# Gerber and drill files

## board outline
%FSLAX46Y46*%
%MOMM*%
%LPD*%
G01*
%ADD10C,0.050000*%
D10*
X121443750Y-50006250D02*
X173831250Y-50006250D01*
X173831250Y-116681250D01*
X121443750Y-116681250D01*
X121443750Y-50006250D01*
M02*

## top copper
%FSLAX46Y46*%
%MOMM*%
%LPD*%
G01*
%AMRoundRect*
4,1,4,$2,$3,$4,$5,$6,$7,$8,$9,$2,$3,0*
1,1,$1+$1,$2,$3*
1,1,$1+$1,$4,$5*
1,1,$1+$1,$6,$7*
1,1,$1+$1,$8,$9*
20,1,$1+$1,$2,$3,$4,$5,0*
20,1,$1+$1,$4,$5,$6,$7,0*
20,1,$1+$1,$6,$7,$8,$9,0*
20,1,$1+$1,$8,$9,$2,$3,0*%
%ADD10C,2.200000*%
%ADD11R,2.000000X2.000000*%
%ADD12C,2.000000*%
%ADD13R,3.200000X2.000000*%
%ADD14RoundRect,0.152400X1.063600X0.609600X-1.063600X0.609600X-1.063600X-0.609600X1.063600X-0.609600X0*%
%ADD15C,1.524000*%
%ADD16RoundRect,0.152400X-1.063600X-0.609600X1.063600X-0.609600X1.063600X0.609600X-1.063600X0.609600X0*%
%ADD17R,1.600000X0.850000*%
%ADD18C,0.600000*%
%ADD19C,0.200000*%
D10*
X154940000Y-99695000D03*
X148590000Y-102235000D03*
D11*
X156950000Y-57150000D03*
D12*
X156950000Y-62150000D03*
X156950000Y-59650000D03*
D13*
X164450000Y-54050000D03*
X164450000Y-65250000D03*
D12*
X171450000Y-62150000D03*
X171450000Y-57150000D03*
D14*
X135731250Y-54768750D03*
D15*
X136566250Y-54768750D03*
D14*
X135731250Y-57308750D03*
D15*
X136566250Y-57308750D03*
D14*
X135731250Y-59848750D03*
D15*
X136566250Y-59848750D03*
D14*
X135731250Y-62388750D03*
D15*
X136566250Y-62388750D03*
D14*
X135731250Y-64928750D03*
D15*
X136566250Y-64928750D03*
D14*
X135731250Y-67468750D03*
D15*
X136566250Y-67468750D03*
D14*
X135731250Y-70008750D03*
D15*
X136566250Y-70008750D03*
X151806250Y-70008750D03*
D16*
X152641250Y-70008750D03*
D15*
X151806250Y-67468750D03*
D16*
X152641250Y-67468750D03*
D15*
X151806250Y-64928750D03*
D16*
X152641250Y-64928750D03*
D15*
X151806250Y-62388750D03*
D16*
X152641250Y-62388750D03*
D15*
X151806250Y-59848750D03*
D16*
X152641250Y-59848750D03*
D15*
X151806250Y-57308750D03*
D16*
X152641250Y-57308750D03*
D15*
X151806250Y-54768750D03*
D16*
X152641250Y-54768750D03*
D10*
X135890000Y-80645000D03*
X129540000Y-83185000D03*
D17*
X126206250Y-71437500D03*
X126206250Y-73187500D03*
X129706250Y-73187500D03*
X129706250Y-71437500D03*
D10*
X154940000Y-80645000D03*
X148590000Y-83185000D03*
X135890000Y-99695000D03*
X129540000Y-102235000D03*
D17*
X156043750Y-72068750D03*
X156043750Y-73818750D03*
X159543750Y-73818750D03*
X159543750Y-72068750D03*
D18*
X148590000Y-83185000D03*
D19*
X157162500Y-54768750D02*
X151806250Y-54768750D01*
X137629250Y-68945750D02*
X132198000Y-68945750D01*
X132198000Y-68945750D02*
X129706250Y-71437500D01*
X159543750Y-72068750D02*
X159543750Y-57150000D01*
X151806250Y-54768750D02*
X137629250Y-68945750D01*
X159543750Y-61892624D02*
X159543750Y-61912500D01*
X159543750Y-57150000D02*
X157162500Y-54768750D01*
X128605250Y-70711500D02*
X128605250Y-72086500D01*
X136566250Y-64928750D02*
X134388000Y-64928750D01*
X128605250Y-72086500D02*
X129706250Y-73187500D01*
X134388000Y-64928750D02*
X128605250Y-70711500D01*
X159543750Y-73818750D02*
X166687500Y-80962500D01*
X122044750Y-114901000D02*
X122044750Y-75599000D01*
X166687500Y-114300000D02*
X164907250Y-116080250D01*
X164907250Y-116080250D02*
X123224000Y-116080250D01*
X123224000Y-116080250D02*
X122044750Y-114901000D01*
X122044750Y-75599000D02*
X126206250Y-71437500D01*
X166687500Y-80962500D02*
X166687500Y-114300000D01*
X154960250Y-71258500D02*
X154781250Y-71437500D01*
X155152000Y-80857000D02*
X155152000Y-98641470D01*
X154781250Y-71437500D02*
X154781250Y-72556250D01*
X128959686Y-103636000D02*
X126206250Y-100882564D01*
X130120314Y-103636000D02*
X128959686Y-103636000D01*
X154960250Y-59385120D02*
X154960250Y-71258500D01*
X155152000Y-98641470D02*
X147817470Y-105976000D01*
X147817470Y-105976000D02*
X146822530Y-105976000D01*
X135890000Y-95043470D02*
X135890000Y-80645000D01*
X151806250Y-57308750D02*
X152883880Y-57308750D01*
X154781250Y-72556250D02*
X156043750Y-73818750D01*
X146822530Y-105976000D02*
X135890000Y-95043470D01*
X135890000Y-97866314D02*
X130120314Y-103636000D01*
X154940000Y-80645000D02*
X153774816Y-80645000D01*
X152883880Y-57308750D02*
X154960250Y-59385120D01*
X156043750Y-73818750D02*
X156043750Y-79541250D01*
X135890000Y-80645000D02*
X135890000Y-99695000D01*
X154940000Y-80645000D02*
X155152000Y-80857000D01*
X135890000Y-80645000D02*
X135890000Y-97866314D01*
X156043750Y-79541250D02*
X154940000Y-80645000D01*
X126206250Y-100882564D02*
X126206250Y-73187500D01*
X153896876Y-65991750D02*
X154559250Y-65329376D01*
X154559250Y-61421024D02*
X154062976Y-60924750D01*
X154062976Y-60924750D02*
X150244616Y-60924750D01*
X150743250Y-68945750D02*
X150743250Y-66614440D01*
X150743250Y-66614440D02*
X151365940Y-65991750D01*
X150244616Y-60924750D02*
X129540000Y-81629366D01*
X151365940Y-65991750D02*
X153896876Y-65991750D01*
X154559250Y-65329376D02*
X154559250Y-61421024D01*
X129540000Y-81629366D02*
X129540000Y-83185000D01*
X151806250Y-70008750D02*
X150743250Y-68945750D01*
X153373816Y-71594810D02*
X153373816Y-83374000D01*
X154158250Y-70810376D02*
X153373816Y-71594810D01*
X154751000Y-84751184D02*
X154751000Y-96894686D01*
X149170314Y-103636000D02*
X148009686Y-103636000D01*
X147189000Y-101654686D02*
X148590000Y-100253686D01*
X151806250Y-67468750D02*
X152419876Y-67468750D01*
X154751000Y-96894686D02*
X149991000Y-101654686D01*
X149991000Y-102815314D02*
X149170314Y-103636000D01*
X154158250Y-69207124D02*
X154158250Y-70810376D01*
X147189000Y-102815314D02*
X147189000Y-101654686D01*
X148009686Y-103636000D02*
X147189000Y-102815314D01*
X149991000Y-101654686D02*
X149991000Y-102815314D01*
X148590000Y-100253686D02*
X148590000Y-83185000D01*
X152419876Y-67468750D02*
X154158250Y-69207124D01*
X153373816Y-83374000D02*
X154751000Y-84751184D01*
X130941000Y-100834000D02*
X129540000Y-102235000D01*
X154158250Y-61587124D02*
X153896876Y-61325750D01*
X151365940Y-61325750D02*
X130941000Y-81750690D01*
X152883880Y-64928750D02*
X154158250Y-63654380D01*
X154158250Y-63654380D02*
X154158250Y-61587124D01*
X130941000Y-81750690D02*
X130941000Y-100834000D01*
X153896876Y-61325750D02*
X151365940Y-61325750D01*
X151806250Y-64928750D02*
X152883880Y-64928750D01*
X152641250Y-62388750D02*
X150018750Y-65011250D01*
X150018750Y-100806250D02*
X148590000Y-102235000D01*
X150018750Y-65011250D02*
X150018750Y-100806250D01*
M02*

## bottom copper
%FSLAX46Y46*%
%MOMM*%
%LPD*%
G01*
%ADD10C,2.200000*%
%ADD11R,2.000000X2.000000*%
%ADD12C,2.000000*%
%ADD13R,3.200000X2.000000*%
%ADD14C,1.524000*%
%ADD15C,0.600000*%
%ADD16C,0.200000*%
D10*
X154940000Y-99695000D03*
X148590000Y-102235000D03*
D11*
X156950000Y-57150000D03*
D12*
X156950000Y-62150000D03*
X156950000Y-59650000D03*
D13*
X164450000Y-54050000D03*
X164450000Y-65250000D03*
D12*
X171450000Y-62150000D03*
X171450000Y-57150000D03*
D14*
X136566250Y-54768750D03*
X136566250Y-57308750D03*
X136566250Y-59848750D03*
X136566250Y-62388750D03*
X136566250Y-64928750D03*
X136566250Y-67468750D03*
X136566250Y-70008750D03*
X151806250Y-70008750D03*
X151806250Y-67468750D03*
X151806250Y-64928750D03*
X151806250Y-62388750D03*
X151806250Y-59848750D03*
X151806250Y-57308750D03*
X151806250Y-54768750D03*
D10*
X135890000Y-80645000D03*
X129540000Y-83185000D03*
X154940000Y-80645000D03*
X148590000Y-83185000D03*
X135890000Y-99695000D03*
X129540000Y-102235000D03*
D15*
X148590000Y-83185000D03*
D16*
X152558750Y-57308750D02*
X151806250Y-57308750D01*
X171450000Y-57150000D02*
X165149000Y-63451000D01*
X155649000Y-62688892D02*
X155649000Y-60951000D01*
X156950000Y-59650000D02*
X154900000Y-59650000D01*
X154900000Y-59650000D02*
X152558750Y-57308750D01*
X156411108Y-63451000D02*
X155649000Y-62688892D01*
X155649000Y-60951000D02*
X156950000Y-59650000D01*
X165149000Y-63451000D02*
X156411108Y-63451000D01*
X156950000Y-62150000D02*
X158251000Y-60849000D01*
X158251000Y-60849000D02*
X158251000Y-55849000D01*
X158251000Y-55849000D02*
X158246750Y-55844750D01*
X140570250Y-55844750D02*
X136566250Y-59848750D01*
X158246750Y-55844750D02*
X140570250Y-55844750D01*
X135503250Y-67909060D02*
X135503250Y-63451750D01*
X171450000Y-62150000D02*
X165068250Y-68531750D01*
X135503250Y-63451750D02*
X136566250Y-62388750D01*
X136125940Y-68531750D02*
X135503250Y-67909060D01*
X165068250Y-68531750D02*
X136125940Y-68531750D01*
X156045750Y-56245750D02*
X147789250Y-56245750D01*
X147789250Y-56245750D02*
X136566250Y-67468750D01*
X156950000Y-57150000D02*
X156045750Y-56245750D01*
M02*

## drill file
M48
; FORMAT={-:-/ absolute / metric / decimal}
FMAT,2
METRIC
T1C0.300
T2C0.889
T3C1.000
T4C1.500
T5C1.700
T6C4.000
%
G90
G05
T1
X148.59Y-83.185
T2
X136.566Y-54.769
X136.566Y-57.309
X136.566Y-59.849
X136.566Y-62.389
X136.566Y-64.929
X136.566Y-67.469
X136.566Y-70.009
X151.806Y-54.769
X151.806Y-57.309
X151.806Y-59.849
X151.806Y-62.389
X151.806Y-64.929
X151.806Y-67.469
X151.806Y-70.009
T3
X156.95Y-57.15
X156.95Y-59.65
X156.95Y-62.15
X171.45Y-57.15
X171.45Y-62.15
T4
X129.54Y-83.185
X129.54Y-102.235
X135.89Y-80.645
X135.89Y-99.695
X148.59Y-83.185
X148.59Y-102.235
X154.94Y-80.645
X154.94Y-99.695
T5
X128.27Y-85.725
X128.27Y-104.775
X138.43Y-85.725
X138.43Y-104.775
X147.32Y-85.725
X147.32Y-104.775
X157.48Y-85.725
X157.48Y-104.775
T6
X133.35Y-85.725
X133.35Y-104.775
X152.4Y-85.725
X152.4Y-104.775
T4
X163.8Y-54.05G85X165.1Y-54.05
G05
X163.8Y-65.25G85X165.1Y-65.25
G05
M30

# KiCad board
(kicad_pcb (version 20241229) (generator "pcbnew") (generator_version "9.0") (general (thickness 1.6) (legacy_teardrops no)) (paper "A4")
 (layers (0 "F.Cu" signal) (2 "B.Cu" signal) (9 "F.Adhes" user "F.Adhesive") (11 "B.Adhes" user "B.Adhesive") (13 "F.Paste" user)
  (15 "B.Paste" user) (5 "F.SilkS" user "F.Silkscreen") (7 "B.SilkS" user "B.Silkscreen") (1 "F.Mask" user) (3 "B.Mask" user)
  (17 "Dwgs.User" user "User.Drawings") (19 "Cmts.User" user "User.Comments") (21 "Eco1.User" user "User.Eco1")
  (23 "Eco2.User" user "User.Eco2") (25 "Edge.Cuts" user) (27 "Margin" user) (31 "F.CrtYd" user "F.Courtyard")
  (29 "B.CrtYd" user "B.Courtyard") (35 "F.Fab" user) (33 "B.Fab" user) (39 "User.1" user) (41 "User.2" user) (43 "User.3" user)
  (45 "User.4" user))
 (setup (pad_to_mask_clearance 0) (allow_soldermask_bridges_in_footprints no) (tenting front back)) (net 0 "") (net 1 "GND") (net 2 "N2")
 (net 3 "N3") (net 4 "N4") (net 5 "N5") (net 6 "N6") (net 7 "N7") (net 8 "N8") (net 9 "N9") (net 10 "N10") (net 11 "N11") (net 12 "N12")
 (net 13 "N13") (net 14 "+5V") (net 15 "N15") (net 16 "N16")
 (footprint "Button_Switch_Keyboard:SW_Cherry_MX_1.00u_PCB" (layer "F.Cu") (at 154.94 99.695)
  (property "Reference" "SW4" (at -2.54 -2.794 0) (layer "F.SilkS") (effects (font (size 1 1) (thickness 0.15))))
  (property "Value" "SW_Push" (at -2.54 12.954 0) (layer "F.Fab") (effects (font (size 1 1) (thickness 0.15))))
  (pad "" np_thru_hole circle (at -7.62 5.08) (size 1.7 1.7) (drill 1.7) (layers "*.Cu" "*.Mask"))
  (pad "" np_thru_hole circle (at -2.54 5.08) (size 4 4) (drill 4) (layers "*.Cu" "*.Mask"))
  (pad "" np_thru_hole circle (at 2.54 5.08) (size 1.7 1.7) (drill 1.7) (layers "*.Cu" "*.Mask"))
  (pad "1" thru_hole circle (at 0 0) (size 2.2 2.2) (drill 1.5) (layers "*.Cu" "*.Mask") (remove_unused_layers no) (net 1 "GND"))
  (pad "2" thru_hole circle (at -6.35 2.54) (size 2.2 2.2) (drill 1.5) (layers "*.Cu" "*.Mask") (remove_unused_layers no) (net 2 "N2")))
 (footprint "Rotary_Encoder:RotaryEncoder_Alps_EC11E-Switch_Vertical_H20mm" (layer "F.Cu") (at 156.95 57.15)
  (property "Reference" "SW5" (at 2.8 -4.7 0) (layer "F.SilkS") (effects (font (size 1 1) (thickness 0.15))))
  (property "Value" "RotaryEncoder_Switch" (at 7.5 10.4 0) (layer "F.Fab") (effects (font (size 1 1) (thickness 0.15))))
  (pad "A" thru_hole rect (at 0 0) (size 2 2) (drill 1) (layers "*.Cu" "*.Mask") (remove_unused_layers no) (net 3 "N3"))
  (pad "B" thru_hole circle (at 0 5) (size 2 2) (drill 1) (layers "*.Cu" "*.Mask") (remove_unused_layers no) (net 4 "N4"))
  (pad "C" thru_hole circle (at 0 2.5) (size 2 2) (drill 1) (layers "*.Cu" "*.Mask") (remove_unused_layers no) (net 1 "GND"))
  (pad "MP" thru_hole rect (at 7.5 -3.1) (size 3.2 2) (drill oval 2.8 1.5) (layers "*.Cu" "*.Mask") (remove_unused_layers no))
  (pad "MP" thru_hole rect (at 7.5 8.1) (size 3.2 2) (drill oval 2.8 1.5) (layers "*.Cu" "*.Mask") (remove_unused_layers no))
  (pad "S1" thru_hole circle (at 14.5 5) (size 2 2) (drill 1) (layers "*.Cu" "*.Mask") (remove_unused_layers no) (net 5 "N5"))
  (pad "S2" thru_hole circle (at 14.5 0) (size 2 2) (drill 1) (layers "*.Cu" "*.Mask") (remove_unused_layers no) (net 1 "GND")))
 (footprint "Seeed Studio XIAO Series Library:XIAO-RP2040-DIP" (layer "F.Cu") (at 144.18625 62.38875)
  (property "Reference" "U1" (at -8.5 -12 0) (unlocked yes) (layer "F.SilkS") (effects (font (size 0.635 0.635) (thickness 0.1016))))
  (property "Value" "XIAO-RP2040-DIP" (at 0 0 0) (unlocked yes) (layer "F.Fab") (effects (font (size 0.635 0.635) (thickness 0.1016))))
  (pad "1" smd roundrect (at -8.455 -7.62 180) (size 2.432 1.524) (layers "F.Cu" "F.Mask") (roundrect_rratio 0.1) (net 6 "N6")
   (thermal_bridge_angle 45))
  (pad "1" thru_hole circle (at -7.62 -7.62 180) (size 1.524 1.524) (drill 0.889) (layers "*.Cu" "*.Mask") (remove_unused_layers no)
   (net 6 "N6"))
  (pad "2" smd roundrect (at -8.455 -5.08 180) (size 2.432 1.524) (layers "F.Cu" "F.Mask") (roundrect_rratio 0.1) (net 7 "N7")
   (thermal_bridge_angle 45))
  (pad "2" thru_hole circle (at -7.62 -5.08 180) (size 1.524 1.524) (drill 0.889) (layers "*.Cu" "*.Mask") (remove_unused_layers no)
   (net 7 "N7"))
  (pad "3" smd roundrect (at -8.455 -2.54 180) (size 2.432 1.524) (layers "F.Cu" "F.Mask") (roundrect_rratio 0.1) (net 4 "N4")
   (thermal_bridge_angle 45))
  (pad "3" thru_hole circle (at -7.62 -2.54 180) (size 1.524 1.524) (drill 0.889) (layers "*.Cu" "*.Mask") (remove_unused_layers no)
   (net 4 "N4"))
  (pad "4" smd roundrect (at -8.455 0 180) (size 2.432 1.524) (layers "F.Cu" "F.Mask") (roundrect_rratio 0.1) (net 5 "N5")
   (thermal_bridge_angle 45))
  (pad "4" thru_hole circle (at -7.62 0 180) (size 1.524 1.524) (drill 0.889) (layers "*.Cu" "*.Mask") (remove_unused_layers no)
   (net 5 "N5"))
  (pad "5" smd roundrect (at -8.455 2.54 180) (size 2.432 1.524) (layers "F.Cu" "F.Mask") (roundrect_rratio 0.1) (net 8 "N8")
   (thermal_bridge_angle 45))
  (pad "5" thru_hole circle (at -7.62 2.54 180) (size 1.524 1.524) (drill 0.889) (layers "*.Cu" "*.Mask") (remove_unused_layers no)
   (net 8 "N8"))
  (pad "6" smd roundrect (at -8.455 5.08 180) (size 2.432 1.524) (layers "F.Cu" "F.Mask") (roundrect_rratio 0.1) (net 3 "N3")
   (thermal_bridge_angle 45))
  (pad "6" thru_hole circle (at -7.62 5.08 180) (size 1.524 1.524) (drill 0.889) (layers "*.Cu" "*.Mask") (remove_unused_layers no)
   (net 3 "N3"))
  (pad "7" smd roundrect (at -8.455 7.62 180) (size 2.432 1.524) (layers "F.Cu" "F.Mask") (roundrect_rratio 0.1) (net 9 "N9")
   (thermal_bridge_angle 45))
  (pad "7" thru_hole circle (at -7.62 7.62 180) (size 1.524 1.524) (drill 0.889) (layers "*.Cu" "*.Mask") (remove_unused_layers no)
   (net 9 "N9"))
  (pad "8" thru_hole circle (at 7.62 7.62) (size 1.524 1.524) (drill 0.889) (layers "*.Cu" "*.Mask") (remove_unused_layers no)
   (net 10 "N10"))
  (pad "8" smd roundrect (at 8.455 7.62) (size 2.432 1.524) (layers "F.Cu" "F.Mask") (roundrect_rratio 0.1) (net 10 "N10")
   (thermal_bridge_angle 45))
  (pad "9" thru_hole circle (at 7.62 5.08) (size 1.524 1.524) (drill 0.889) (layers "*.Cu" "*.Mask") (remove_unused_layers no)
   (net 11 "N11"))
  (pad "9" smd roundrect (at 8.455 5.08) (size 2.432 1.524) (layers "F.Cu" "F.Mask") (roundrect_rratio 0.1) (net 11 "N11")
   (thermal_bridge_angle 45))
  (pad "10" thru_hole circle (at 7.62 2.54) (size 1.524 1.524) (drill 0.889) (layers "*.Cu" "*.Mask") (remove_unused_layers no)
   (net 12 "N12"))
  (pad "10" smd roundrect (at 8.455 2.54) (size 2.432 1.524) (layers "F.Cu" "F.Mask") (roundrect_rratio 0.1) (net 12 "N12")
   (thermal_bridge_angle 45))
  (pad "11" thru_hole circle (at 7.62 0) (size 1.524 1.524) (drill 0.889) (layers "*.Cu" "*.Mask") (remove_unused_layers no) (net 2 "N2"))
  (pad "11" smd roundrect (at 8.455 0) (size 2.432 1.524) (layers "F.Cu" "F.Mask") (roundrect_rratio 0.1) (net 2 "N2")
   (thermal_bridge_angle 45))
  (pad "12" thru_hole circle (at 7.62 -2.54) (size 1.524 1.524) (drill 0.889) (layers "*.Cu" "*.Mask") (remove_unused_layers no)
   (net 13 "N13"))
  (pad "12" smd roundrect (at 8.455 -2.54) (size 2.432 1.524) (layers "F.Cu" "F.Mask") (roundrect_rratio 0.1) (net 13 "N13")
   (thermal_bridge_angle 45))
  (pad "13" thru_hole circle (at 7.62 -5.08) (size 1.524 1.524) (drill 0.889) (layers "*.Cu" "*.Mask") (remove_unused_layers no)
   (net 1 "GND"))
  (pad "13" smd roundrect (at 8.455 -5.08) (size 2.432 1.524) (layers "F.Cu" "F.Mask") (roundrect_rratio 0.1) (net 1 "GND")
   (thermal_bridge_angle 45))
  (pad "14" thru_hole circle (at 7.62 -7.62) (size 1.524 1.524) (drill 0.889) (layers "*.Cu" "*.Mask") (remove_unused_layers no)
   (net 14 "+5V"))
  (pad "14" smd roundrect (at 8.455 -7.62) (size 2.432 1.524) (layers "F.Cu" "F.Mask") (roundrect_rratio 0.1) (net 14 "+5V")
   (thermal_bridge_angle 45)))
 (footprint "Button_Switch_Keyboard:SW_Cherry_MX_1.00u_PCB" (layer "F.Cu") (at 135.89 80.645)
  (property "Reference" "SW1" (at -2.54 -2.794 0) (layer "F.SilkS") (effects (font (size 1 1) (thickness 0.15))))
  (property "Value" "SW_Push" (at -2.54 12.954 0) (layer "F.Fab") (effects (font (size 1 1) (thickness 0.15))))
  (pad "" np_thru_hole circle (at -7.62 5.08) (size 1.7 1.7) (drill 1.7) (layers "*.Cu" "*.Mask"))
  (pad "" np_thru_hole circle (at -2.54 5.08) (size 4 4) (drill 4) (layers "*.Cu" "*.Mask"))
  (pad "" np_thru_hole circle (at 2.54 5.08) (size 1.7 1.7) (drill 1.7) (layers "*.Cu" "*.Mask"))
  (pad "1" thru_hole circle (at 0 0) (size 2.2 2.2) (drill 1.5) (layers "*.Cu" "*.Mask") (remove_unused_layers no) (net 1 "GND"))
  (pad "2" thru_hole circle (at -6.35 2.54) (size 2.2 2.2) (drill 1.5) (layers "*.Cu" "*.Mask") (remove_unused_layers no) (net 10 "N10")))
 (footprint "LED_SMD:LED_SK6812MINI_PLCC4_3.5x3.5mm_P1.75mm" (layer "F.Cu") (at 127.95625 72.3125)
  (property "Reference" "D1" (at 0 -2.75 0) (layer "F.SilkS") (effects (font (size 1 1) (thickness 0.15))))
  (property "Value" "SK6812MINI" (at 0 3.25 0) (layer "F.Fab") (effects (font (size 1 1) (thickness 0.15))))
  (pad "1" smd rect (at -1.75 -0.875) (size 1.6 0.85) (layers "F.Cu" "F.Mask" "F.Paste") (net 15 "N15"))
  (pad "2" smd rect (at -1.75 0.875) (size 1.6 0.85) (layers "F.Cu" "F.Mask" "F.Paste") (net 1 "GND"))
  (pad "3" smd rect (at 1.75 0.875) (size 1.6 0.85) (layers "F.Cu" "F.Mask" "F.Paste") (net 8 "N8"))
  (pad "4" smd rect (at 1.75 -0.875) (size 1.6 0.85) (layers "F.Cu" "F.Mask" "F.Paste") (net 14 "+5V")))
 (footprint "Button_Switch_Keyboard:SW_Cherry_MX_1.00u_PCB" (layer "F.Cu") (at 154.94 80.645)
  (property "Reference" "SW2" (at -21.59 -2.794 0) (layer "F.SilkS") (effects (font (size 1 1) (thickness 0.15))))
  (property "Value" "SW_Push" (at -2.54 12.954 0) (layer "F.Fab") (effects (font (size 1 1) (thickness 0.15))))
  (pad "" np_thru_hole circle (at -7.62 5.08) (size 1.7 1.7) (drill 1.7) (layers "*.Cu" "*.Mask"))
  (pad "" np_thru_hole circle (at -2.54 5.08) (size 4 4) (drill 4) (layers "*.Cu" "*.Mask"))
  (pad "" np_thru_hole circle (at 2.54 5.08) (size 1.7 1.7) (drill 1.7) (layers "*.Cu" "*.Mask"))
  (pad "1" thru_hole circle (at 0 0) (size 2.2 2.2) (drill 1.5) (layers "*.Cu" "*.Mask") (remove_unused_layers no) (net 1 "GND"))
  (pad "2" thru_hole circle (at -6.35 2.54) (size 2.2 2.2) (drill 1.5) (layers "*.Cu" "*.Mask") (remove_unused_layers no) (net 11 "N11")))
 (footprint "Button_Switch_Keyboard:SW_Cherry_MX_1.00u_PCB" (layer "F.Cu") (at 135.89 99.695)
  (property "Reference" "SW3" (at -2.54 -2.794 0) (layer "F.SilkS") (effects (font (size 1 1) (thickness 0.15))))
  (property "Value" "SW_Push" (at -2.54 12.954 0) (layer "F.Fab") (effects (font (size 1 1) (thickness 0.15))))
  (pad "" np_thru_hole circle (at -7.62 5.08) (size 1.7 1.7) (drill 1.7) (layers "*.Cu" "*.Mask"))
  (pad "" np_thru_hole circle (at -2.54 5.08) (size 4 4) (drill 4) (layers "*.Cu" "*.Mask"))
  (pad "" np_thru_hole circle (at 2.54 5.08) (size 1.7 1.7) (drill 1.7) (layers "*.Cu" "*.Mask"))
  (pad "1" thru_hole circle (at 0 0) (size 2.2 2.2) (drill 1.5) (layers "*.Cu" "*.Mask") (remove_unused_layers no) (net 1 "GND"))
  (pad "2" thru_hole circle (at -6.35 2.54) (size 2.2 2.2) (drill 1.5) (layers "*.Cu" "*.Mask") (remove_unused_layers no) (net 12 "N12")))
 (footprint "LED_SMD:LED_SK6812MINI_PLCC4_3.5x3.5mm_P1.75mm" (layer "F.Cu") (at 157.79375 72.94375)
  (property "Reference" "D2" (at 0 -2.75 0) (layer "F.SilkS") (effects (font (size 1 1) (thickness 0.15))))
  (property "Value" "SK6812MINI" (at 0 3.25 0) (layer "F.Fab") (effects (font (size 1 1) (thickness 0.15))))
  (pad "1" smd rect (at -1.75 -0.875) (size 1.6 0.85) (layers "F.Cu" "F.Mask" "F.Paste") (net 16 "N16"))
  (pad "2" smd rect (at -1.75 0.875) (size 1.6 0.85) (layers "F.Cu" "F.Mask" "F.Paste") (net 1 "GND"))
  (pad "3" smd rect (at 1.75 0.875) (size 1.6 0.85) (layers "F.Cu" "F.Mask" "F.Paste") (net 15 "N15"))
  (pad "4" smd rect (at 1.75 -0.875) (size 1.6 0.85) (layers "F.Cu" "F.Mask" "F.Paste") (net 14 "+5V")))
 (gr_rect (start 121.44375 50.00625) (end 173.83125 116.68125) (stroke (width 0.05) (type default)) (fill no) (layer "Edge.Cuts"))
 (segment (start 157.1625 54.76875) (end 151.80625 54.76875) (width 0.2) (layer "F.Cu") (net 14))
 (segment (start 137.62925 68.94575) (end 132.198 68.94575) (width 0.2) (layer "F.Cu") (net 14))
 (segment (start 132.198 68.94575) (end 129.70625 71.4375) (width 0.2) (layer "F.Cu") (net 14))
 (segment (start 159.54375 72.06875) (end 159.54375 57.15) (width 0.2) (layer "F.Cu") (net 14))
 (segment (start 151.80625 54.76875) (end 137.62925 68.94575) (width 0.2) (layer "F.Cu") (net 14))
 (segment (start 159.54375 61.892624) (end 159.54375 61.9125) (width 0.2) (layer "F.Cu") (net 14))
 (segment (start 159.54375 57.15) (end 157.1625 54.76875) (width 0.2) (layer "F.Cu") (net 14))
 (segment (start 128.60525 70.7115) (end 128.60525 72.0865) (width 0.2) (layer "F.Cu") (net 8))
 (segment (start 136.56625 64.92875) (end 134.388 64.92875) (width 0.2) (layer "F.Cu") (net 8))
 (segment (start 128.60525 72.0865) (end 129.70625 73.1875) (width 0.2) (layer "F.Cu") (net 8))
 (segment (start 134.388 64.92875) (end 128.60525 70.7115) (width 0.2) (layer "F.Cu") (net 8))
 (segment (start 159.54375 73.81875) (end 166.6875 80.9625) (width 0.2) (layer "F.Cu") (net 15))
 (segment (start 122.04475 114.901) (end 122.04475 75.599) (width 0.2) (layer "F.Cu") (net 15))
 (segment (start 166.6875 114.3) (end 164.90725 116.08025) (width 0.2) (layer "F.Cu") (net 15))
 (segment (start 164.90725 116.08025) (end 123.224 116.08025) (width 0.2) (layer "F.Cu") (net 15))
 (segment (start 123.224 116.08025) (end 122.04475 114.901) (width 0.2) (layer "F.Cu") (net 15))
 (segment (start 122.04475 75.599) (end 126.20625 71.4375) (width 0.2) (layer "F.Cu") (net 15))
 (segment (start 166.6875 80.9625) (end 166.6875 114.3) (width 0.2) (layer "F.Cu") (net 15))
 (segment (start 154.96025 71.2585) (end 154.78125 71.4375) (width 0.2) (layer "F.Cu") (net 1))
 (segment (start 155.152 80.857) (end 155.152 98.64147) (width 0.2) (layer "F.Cu") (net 1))
 (segment (start 154.78125 71.4375) (end 154.78125 72.55625) (width 0.2) (layer "F.Cu") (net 1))
 (segment (start 128.959686 103.636) (end 126.20625 100.882564) (width 0.2) (layer "F.Cu") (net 1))
 (segment (start 130.120314 103.636) (end 128.959686 103.636) (width 0.2) (layer "F.Cu") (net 1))
 (segment (start 154.96025 59.38512) (end 154.96025 71.2585) (width 0.2) (layer "F.Cu") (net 1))
 (segment (start 155.152 98.64147) (end 147.81747 105.976) (width 0.2) (layer "F.Cu") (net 1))
 (segment (start 147.81747 105.976) (end 146.82253 105.976) (width 0.2) (layer "F.Cu") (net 1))
 (segment (start 135.89 95.04347) (end 135.89 80.645) (width 0.2) (layer "F.Cu") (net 1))
 (segment (start 151.80625 57.30875) (end 152.88388 57.30875) (width 0.2) (layer "F.Cu") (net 1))
 (segment (start 154.78125 72.55625) (end 156.04375 73.81875) (width 0.2) (layer "F.Cu") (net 1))
 (segment (start 146.82253 105.976) (end 135.89 95.04347) (width 0.2) (layer "F.Cu") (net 1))
 (segment (start 135.89 97.866314) (end 130.120314 103.636) (width 0.2) (layer "F.Cu") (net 1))
 (segment (start 154.94 80.645) (end 153.774816 80.645) (width 0.2) (layer "F.Cu") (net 1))
 (segment (start 152.88388 57.30875) (end 154.96025 59.38512) (width 0.2) (layer "F.Cu") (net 1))
 (segment (start 156.04375 73.81875) (end 156.04375 79.54125) (width 0.2) (layer "F.Cu") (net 1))
 (segment (start 135.89 80.645) (end 135.89 99.695) (width 0.2) (layer "F.Cu") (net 1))
 (segment (start 154.94 80.645) (end 155.152 80.857) (width 0.2) (layer "F.Cu") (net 1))
 (segment (start 135.89 80.645) (end 135.89 97.866314) (width 0.2) (layer "F.Cu") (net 1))
 (segment (start 156.04375 79.54125) (end 154.94 80.645) (width 0.2) (layer "F.Cu") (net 1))
 (segment (start 126.20625 100.882564) (end 126.20625 73.1875) (width 0.2) (layer "F.Cu") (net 1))
 (segment (start 152.55875 57.30875) (end 151.80625 57.30875) (width 0.2) (layer "B.Cu") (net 1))
 (segment (start 171.45 57.15) (end 165.149 63.451) (width 0.2) (layer "B.Cu") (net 1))
 (segment (start 155.649 62.688892) (end 155.649 60.951) (width 0.2) (layer "B.Cu") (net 1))
 (segment (start 156.95 59.65) (end 154.9 59.65) (width 0.2) (layer "B.Cu") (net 1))
 (segment (start 154.9 59.65) (end 152.55875 57.30875) (width 0.2) (layer "B.Cu") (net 1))
 (segment (start 156.411108 63.451) (end 155.649 62.688892) (width 0.2) (layer "B.Cu") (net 1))
 (segment (start 155.649 60.951) (end 156.95 59.65) (width 0.2) (layer "B.Cu") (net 1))
 (segment (start 165.149 63.451) (end 156.411108 63.451) (width 0.2) (layer "B.Cu") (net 1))
 (segment (start 153.896876 65.99175) (end 154.55925 65.329376) (width 0.2) (layer "F.Cu") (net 10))
 (segment (start 154.55925 61.421024) (end 154.062976 60.92475) (width 0.2) (layer "F.Cu") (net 10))
 (segment (start 154.062976 60.92475) (end 150.244616 60.92475) (width 0.2) (layer "F.Cu") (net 10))
 (segment (start 150.74325 68.94575) (end 150.74325 66.61444) (width 0.2) (layer "F.Cu") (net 10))
 (segment (start 150.74325 66.61444) (end 151.36594 65.99175) (width 0.2) (layer "F.Cu") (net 10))
 (segment (start 150.244616 60.92475) (end 129.54 81.629366) (width 0.2) (layer "F.Cu") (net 10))
 (segment (start 151.36594 65.99175) (end 153.896876 65.99175) (width 0.2) (layer "F.Cu") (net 10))
 (segment (start 154.55925 65.329376) (end 154.55925 61.421024) (width 0.2) (layer "F.Cu") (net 10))
 (segment (start 129.54 81.629366) (end 129.54 83.185) (width 0.2) (layer "F.Cu") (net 10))
 (segment (start 151.80625 70.00875) (end 150.74325 68.94575) (width 0.2) (layer "F.Cu") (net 10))
 (segment (start 153.373816 71.59481) (end 153.373816 83.374) (width 0.2) (layer "F.Cu") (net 11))
 (segment (start 154.15825 70.810376) (end 153.373816 71.59481) (width 0.2) (layer "F.Cu") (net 11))
 (segment (start 154.751 84.751184) (end 154.751 96.894686) (width 0.2) (layer "F.Cu") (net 11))
 (segment (start 149.170314 103.636) (end 148.009686 103.636) (width 0.2) (layer "F.Cu") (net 11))
 (segment (start 147.189 101.654686) (end 148.59 100.253686) (width 0.2) (layer "F.Cu") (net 11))
 (segment (start 151.80625 67.46875) (end 152.419876 67.46875) (width 0.2) (layer "F.Cu") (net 11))
 (segment (start 154.751 96.894686) (end 149.991 101.654686) (width 0.2) (layer "F.Cu") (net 11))
 (segment (start 149.991 102.815314) (end 149.170314 103.636) (width 0.2) (layer "F.Cu") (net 11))
 (segment (start 154.15825 69.207124) (end 154.15825 70.810376) (width 0.2) (layer "F.Cu") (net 11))
 (segment (start 147.189 102.815314) (end 147.189 101.654686) (width 0.2) (layer "F.Cu") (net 11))
 (segment (start 148.009686 103.636) (end 147.189 102.815314) (width 0.2) (layer "F.Cu") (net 11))
 (segment (start 149.991 101.654686) (end 149.991 102.815314) (width 0.2) (layer "F.Cu") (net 11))
 (segment (start 148.59 100.253686) (end 148.59 83.185) (width 0.2) (layer "F.Cu") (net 11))
 (segment (start 152.419876 67.46875) (end 154.15825 69.207124) (width 0.2) (layer "F.Cu") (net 11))
 (segment (start 153.373816 83.374) (end 154.751 84.751184) (width 0.2) (layer "F.Cu") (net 11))
 (via (at 148.59 83.185) (size 0.6) (drill 0.3) (layers "F.Cu" "B.Cu") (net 11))
 (segment (start 130.941 100.834) (end 129.54 102.235) (width 0.2) (layer "F.Cu") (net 12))
 (segment (start 154.15825 61.587124) (end 153.896876 61.32575) (width 0.2) (layer "F.Cu") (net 12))
 (segment (start 151.36594 61.32575) (end 130.941 81.75069) (width 0.2) (layer "F.Cu") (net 12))
 (segment (start 152.88388 64.92875) (end 154.15825 63.65438) (width 0.2) (layer "F.Cu") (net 12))
 (segment (start 154.15825 63.65438) (end 154.15825 61.587124) (width 0.2) (layer "F.Cu") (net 12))
 (segment (start 130.941 81.75069) (end 130.941 100.834) (width 0.2) (layer "F.Cu") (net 12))
 (segment (start 153.896876 61.32575) (end 151.36594 61.32575) (width 0.2) (layer "F.Cu") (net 12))
 (segment (start 151.80625 64.92875) (end 152.88388 64.92875) (width 0.2) (layer "F.Cu") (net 12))
 (segment (start 152.64125 62.38875) (end 150.01875 65.01125) (width 0.2) (layer "F.Cu") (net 2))
 (segment (start 150.01875 100.80625) (end 148.59 102.235) (width 0.2) (layer "F.Cu") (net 2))
 (segment (start 150.01875 65.01125) (end 150.01875 100.80625) (width 0.2) (layer "F.Cu") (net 2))
 (segment (start 156.95 62.15) (end 158.251 60.849) (width 0.2) (layer "B.Cu") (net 4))
 (segment (start 158.251 60.849) (end 158.251 55.849) (width 0.2) (layer "B.Cu") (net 4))
 (segment (start 158.251 55.849) (end 158.24675 55.84475) (width 0.2) (layer "B.Cu") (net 4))
 (segment (start 140.57025 55.84475) (end 136.56625 59.84875) (width 0.2) (layer "B.Cu") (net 4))
 (segment (start 158.24675 55.84475) (end 140.57025 55.84475) (width 0.2) (layer "B.Cu") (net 4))
 (segment (start 135.50325 67.90906) (end 135.50325 63.45175) (width 0.2) (layer "B.Cu") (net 5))
 (segment (start 171.45 62.15) (end 165.06825 68.53175) (width 0.2) (layer "B.Cu") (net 5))
 (segment (start 135.50325 63.45175) (end 136.56625 62.38875) (width 0.2) (layer "B.Cu") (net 5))
 (segment (start 136.12594 68.53175) (end 135.50325 67.90906) (width 0.2) (layer "B.Cu") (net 5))
 (segment (start 165.06825 68.53175) (end 136.12594 68.53175) (width 0.2) (layer "B.Cu") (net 5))
 (segment (start 156.04575 56.24575) (end 147.78925 56.24575) (width 0.2) (layer "B.Cu") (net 3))
 (segment (start 147.78925 56.24575) (end 136.56625 67.46875) (width 0.2) (layer "B.Cu") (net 3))
 (segment (start 156.95 57.15) (end 156.04575 56.24575) (width 0.2) (layer "B.Cu") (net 3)))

